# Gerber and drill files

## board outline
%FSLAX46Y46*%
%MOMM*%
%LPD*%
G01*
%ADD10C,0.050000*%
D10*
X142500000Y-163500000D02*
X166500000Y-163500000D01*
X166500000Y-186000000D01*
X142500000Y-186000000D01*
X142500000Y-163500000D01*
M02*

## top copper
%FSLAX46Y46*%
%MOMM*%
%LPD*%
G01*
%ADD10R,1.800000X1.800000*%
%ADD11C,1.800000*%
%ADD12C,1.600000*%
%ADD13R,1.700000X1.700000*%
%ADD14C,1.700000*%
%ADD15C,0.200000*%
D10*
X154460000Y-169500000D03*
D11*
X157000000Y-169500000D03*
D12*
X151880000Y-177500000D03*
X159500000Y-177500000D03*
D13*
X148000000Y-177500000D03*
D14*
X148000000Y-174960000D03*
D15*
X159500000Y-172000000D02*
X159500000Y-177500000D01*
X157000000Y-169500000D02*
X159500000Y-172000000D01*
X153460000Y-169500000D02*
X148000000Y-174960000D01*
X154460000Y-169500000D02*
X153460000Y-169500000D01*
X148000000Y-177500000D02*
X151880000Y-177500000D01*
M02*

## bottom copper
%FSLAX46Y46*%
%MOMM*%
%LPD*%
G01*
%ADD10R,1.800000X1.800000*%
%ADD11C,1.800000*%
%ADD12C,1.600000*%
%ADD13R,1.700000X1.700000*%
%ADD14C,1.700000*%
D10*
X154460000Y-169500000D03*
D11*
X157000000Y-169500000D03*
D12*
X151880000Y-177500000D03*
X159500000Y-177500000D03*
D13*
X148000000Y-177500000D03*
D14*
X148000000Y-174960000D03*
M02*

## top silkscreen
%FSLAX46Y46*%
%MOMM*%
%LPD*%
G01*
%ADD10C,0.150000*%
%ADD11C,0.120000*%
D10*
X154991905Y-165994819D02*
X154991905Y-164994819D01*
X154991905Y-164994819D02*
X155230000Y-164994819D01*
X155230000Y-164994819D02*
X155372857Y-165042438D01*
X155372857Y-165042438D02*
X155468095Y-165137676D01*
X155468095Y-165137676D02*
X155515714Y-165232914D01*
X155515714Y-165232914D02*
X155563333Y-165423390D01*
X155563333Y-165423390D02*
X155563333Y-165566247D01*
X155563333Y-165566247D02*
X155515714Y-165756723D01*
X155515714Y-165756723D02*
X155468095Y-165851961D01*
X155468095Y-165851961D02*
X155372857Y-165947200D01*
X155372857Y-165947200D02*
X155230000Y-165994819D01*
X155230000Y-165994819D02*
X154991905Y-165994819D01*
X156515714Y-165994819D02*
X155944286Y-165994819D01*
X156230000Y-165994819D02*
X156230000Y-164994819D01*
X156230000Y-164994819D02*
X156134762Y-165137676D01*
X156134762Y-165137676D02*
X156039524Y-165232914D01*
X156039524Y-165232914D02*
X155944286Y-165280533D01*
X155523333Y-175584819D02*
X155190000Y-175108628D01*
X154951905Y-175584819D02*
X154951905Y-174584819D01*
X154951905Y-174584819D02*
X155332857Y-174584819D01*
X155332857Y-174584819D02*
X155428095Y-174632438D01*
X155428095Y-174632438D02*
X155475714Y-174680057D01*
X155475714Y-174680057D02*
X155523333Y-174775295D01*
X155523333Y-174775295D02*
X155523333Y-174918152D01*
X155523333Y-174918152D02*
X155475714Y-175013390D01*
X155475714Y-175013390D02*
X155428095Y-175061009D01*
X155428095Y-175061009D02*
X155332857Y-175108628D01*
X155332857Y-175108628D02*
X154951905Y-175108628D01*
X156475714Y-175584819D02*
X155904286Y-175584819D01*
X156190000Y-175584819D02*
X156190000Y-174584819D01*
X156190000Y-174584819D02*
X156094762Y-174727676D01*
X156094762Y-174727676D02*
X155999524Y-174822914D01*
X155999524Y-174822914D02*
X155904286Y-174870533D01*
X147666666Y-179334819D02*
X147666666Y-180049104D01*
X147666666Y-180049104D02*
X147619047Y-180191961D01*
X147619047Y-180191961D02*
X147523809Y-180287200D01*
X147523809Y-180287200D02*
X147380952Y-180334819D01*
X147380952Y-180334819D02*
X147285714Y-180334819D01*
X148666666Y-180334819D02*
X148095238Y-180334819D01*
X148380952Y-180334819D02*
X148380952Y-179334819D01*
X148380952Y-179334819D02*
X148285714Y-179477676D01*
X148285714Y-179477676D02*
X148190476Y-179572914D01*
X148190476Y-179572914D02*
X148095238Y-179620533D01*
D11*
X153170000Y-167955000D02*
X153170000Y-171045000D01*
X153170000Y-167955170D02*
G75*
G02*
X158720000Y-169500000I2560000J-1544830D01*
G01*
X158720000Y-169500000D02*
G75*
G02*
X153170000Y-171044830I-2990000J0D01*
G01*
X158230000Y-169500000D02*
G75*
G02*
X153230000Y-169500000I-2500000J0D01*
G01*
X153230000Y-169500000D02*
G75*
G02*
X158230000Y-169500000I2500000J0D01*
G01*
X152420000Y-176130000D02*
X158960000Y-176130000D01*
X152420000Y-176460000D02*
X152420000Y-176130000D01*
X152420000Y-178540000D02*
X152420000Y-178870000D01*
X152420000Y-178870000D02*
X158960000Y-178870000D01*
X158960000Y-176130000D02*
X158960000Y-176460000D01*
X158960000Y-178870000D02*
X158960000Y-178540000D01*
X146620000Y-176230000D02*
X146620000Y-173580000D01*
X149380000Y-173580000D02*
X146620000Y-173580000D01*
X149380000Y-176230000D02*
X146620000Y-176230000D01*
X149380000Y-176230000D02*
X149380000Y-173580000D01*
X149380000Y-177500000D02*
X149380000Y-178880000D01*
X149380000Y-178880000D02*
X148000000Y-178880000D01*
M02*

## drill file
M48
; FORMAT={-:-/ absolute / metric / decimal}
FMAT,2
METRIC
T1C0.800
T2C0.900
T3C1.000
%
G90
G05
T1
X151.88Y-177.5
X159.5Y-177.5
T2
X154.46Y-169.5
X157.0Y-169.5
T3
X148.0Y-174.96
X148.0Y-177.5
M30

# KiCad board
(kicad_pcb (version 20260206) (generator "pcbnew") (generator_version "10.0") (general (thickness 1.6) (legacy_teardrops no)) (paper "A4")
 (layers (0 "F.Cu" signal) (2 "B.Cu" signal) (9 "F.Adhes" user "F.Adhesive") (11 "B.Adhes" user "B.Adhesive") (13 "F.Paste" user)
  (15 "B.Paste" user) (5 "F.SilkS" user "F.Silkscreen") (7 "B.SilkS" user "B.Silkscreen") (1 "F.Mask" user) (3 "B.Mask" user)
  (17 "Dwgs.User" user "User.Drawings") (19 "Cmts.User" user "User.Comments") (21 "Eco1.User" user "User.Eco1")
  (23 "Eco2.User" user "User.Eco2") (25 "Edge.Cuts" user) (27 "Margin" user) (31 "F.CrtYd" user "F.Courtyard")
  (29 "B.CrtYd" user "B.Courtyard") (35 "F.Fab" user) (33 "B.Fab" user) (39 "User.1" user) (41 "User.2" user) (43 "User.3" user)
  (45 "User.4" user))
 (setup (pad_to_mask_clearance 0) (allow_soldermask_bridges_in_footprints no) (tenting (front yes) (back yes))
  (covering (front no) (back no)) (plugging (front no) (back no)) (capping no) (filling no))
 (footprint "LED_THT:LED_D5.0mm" (layer "F.Cu") (at 154.46 169.5)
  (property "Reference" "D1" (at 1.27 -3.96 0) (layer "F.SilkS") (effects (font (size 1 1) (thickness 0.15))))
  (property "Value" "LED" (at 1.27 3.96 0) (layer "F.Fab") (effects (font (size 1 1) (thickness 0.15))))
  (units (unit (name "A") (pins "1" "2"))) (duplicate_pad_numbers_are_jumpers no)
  (fp_line (start -1.29 -1.545) (end -1.29 1.545) (stroke (width 0.12) (type solid)) (layer "F.SilkS"))
  (fp_arc (start -1.29 -1.54483) (mid 2.071779 -2.880495) (end 4.26 0) (stroke (width 0.12) (type solid)) (layer "F.SilkS"))
  (fp_arc (start 4.26 0) (mid 2.071779 2.880495) (end -1.29 1.54483) (stroke (width 0.12) (type solid)) (layer "F.SilkS"))
  (fp_circle (center 1.27 0) (end 3.77 0) (stroke (width 0.12) (type solid)) (fill no) (layer "F.SilkS"))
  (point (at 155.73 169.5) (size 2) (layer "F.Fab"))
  (pad "1" thru_hole rect (at 0 0) (size 1.8 1.8) (drill 0.9) (layers "*.Cu" "*.Mask") (remove_unused_layers no) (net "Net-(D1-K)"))
  (pad "2" thru_hole circle (at 2.54 0) (size 1.8 1.8) (drill 0.9) (layers "*.Cu" "*.Mask") (remove_unused_layers no) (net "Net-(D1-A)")))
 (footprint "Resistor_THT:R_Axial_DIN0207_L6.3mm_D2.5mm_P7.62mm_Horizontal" (layer "F.Cu") (at 151.88 177.5)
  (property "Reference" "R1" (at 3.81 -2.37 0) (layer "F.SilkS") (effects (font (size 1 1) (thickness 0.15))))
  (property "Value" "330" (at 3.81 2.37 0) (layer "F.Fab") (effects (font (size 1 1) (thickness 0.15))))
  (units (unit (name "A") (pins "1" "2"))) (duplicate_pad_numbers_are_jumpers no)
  (fp_line (start 0.54 -1.37) (end 7.08 -1.37) (stroke (width 0.12) (type solid)) (layer "F.SilkS"))
  (fp_line (start 0.54 -1.04) (end 0.54 -1.37) (stroke (width 0.12) (type solid)) (layer "F.SilkS"))
  (fp_line (start 0.54 1.04) (end 0.54 1.37) (stroke (width 0.12) (type solid)) (layer "F.SilkS"))
  (fp_line (start 0.54 1.37) (end 7.08 1.37) (stroke (width 0.12) (type solid)) (layer "F.SilkS"))
  (fp_line (start 7.08 -1.37) (end 7.08 -1.04) (stroke (width 0.12) (type solid)) (layer "F.SilkS"))
  (fp_line (start 7.08 1.37) (end 7.08 1.04) (stroke (width 0.12) (type solid)) (layer "F.SilkS"))
  (pad "1" thru_hole circle (at 0 0) (size 1.6 1.6) (drill 0.8) (layers "*.Cu" "*.Mask") (remove_unused_layers no) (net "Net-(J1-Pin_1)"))
  (pad "2" thru_hole circle (at 7.62 0) (size 1.6 1.6) (drill 0.8) (layers "*.Cu" "*.Mask") (remove_unused_layers no) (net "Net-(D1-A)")))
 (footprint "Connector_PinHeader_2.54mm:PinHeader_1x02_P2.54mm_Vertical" (layer "F.Cu") (at 148 177.5 180)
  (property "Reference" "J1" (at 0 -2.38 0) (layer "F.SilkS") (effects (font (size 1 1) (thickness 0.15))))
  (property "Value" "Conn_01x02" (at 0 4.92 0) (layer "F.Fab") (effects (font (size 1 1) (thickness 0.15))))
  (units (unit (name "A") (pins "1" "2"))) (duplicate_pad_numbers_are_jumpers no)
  (fp_line (start 1.38 1.27) (end 1.38 3.92) (stroke (width 0.12) (type solid)) (layer "F.SilkS"))
  (fp_line (start -1.38 3.92) (end 1.38 3.92) (stroke (width 0.12) (type solid)) (layer "F.SilkS"))
  (fp_line (start -1.38 1.27) (end 1.38 1.27) (stroke (width 0.12) (type solid)) (layer "F.SilkS"))
  (fp_line (start -1.38 1.27) (end -1.38 3.92) (stroke (width 0.12) (type solid)) (layer "F.SilkS"))
  (fp_line (start -1.38 0) (end -1.38 -1.38) (stroke (width 0.12) (type solid)) (layer "F.SilkS"))
  (fp_line (start -1.38 -1.38) (end 0 -1.38) (stroke (width 0.12) (type solid)) (layer "F.SilkS"))
  (pad "1" thru_hole rect (at 0 0 180) (size 1.7 1.7) (drill 1) (layers "*.Cu" "*.Mask") (remove_unused_layers no) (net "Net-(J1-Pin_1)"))
  (pad "2" thru_hole circle (at 0 2.54 180) (size 1.7 1.7) (drill 1) (layers "*.Cu" "*.Mask") (remove_unused_layers no) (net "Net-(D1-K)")))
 (gr_rect (start 142.5 163.5) (end 166.5 186) (stroke (width 0.05) (type default)) (fill no) (layer "Edge.Cuts"))
 (segment (start 159.5 172) (end 159.5 177.5) (width 0.2) (layer "F.Cu") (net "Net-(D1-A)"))
 (segment (start 157 169.5) (end 159.5 172) (width 0.2) (layer "F.Cu") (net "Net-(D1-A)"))
 (segment (start 153.46 169.5) (end 148 174.96) (width 0.2) (layer "F.Cu") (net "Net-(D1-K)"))
 (segment (start 154.46 169.5) (end 153.46 169.5) (width 0.2) (layer "F.Cu") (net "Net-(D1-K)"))
 (segment (start 148 177.5) (end 151.88 177.5) (width 0.2) (layer "F.Cu") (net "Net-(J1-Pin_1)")))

